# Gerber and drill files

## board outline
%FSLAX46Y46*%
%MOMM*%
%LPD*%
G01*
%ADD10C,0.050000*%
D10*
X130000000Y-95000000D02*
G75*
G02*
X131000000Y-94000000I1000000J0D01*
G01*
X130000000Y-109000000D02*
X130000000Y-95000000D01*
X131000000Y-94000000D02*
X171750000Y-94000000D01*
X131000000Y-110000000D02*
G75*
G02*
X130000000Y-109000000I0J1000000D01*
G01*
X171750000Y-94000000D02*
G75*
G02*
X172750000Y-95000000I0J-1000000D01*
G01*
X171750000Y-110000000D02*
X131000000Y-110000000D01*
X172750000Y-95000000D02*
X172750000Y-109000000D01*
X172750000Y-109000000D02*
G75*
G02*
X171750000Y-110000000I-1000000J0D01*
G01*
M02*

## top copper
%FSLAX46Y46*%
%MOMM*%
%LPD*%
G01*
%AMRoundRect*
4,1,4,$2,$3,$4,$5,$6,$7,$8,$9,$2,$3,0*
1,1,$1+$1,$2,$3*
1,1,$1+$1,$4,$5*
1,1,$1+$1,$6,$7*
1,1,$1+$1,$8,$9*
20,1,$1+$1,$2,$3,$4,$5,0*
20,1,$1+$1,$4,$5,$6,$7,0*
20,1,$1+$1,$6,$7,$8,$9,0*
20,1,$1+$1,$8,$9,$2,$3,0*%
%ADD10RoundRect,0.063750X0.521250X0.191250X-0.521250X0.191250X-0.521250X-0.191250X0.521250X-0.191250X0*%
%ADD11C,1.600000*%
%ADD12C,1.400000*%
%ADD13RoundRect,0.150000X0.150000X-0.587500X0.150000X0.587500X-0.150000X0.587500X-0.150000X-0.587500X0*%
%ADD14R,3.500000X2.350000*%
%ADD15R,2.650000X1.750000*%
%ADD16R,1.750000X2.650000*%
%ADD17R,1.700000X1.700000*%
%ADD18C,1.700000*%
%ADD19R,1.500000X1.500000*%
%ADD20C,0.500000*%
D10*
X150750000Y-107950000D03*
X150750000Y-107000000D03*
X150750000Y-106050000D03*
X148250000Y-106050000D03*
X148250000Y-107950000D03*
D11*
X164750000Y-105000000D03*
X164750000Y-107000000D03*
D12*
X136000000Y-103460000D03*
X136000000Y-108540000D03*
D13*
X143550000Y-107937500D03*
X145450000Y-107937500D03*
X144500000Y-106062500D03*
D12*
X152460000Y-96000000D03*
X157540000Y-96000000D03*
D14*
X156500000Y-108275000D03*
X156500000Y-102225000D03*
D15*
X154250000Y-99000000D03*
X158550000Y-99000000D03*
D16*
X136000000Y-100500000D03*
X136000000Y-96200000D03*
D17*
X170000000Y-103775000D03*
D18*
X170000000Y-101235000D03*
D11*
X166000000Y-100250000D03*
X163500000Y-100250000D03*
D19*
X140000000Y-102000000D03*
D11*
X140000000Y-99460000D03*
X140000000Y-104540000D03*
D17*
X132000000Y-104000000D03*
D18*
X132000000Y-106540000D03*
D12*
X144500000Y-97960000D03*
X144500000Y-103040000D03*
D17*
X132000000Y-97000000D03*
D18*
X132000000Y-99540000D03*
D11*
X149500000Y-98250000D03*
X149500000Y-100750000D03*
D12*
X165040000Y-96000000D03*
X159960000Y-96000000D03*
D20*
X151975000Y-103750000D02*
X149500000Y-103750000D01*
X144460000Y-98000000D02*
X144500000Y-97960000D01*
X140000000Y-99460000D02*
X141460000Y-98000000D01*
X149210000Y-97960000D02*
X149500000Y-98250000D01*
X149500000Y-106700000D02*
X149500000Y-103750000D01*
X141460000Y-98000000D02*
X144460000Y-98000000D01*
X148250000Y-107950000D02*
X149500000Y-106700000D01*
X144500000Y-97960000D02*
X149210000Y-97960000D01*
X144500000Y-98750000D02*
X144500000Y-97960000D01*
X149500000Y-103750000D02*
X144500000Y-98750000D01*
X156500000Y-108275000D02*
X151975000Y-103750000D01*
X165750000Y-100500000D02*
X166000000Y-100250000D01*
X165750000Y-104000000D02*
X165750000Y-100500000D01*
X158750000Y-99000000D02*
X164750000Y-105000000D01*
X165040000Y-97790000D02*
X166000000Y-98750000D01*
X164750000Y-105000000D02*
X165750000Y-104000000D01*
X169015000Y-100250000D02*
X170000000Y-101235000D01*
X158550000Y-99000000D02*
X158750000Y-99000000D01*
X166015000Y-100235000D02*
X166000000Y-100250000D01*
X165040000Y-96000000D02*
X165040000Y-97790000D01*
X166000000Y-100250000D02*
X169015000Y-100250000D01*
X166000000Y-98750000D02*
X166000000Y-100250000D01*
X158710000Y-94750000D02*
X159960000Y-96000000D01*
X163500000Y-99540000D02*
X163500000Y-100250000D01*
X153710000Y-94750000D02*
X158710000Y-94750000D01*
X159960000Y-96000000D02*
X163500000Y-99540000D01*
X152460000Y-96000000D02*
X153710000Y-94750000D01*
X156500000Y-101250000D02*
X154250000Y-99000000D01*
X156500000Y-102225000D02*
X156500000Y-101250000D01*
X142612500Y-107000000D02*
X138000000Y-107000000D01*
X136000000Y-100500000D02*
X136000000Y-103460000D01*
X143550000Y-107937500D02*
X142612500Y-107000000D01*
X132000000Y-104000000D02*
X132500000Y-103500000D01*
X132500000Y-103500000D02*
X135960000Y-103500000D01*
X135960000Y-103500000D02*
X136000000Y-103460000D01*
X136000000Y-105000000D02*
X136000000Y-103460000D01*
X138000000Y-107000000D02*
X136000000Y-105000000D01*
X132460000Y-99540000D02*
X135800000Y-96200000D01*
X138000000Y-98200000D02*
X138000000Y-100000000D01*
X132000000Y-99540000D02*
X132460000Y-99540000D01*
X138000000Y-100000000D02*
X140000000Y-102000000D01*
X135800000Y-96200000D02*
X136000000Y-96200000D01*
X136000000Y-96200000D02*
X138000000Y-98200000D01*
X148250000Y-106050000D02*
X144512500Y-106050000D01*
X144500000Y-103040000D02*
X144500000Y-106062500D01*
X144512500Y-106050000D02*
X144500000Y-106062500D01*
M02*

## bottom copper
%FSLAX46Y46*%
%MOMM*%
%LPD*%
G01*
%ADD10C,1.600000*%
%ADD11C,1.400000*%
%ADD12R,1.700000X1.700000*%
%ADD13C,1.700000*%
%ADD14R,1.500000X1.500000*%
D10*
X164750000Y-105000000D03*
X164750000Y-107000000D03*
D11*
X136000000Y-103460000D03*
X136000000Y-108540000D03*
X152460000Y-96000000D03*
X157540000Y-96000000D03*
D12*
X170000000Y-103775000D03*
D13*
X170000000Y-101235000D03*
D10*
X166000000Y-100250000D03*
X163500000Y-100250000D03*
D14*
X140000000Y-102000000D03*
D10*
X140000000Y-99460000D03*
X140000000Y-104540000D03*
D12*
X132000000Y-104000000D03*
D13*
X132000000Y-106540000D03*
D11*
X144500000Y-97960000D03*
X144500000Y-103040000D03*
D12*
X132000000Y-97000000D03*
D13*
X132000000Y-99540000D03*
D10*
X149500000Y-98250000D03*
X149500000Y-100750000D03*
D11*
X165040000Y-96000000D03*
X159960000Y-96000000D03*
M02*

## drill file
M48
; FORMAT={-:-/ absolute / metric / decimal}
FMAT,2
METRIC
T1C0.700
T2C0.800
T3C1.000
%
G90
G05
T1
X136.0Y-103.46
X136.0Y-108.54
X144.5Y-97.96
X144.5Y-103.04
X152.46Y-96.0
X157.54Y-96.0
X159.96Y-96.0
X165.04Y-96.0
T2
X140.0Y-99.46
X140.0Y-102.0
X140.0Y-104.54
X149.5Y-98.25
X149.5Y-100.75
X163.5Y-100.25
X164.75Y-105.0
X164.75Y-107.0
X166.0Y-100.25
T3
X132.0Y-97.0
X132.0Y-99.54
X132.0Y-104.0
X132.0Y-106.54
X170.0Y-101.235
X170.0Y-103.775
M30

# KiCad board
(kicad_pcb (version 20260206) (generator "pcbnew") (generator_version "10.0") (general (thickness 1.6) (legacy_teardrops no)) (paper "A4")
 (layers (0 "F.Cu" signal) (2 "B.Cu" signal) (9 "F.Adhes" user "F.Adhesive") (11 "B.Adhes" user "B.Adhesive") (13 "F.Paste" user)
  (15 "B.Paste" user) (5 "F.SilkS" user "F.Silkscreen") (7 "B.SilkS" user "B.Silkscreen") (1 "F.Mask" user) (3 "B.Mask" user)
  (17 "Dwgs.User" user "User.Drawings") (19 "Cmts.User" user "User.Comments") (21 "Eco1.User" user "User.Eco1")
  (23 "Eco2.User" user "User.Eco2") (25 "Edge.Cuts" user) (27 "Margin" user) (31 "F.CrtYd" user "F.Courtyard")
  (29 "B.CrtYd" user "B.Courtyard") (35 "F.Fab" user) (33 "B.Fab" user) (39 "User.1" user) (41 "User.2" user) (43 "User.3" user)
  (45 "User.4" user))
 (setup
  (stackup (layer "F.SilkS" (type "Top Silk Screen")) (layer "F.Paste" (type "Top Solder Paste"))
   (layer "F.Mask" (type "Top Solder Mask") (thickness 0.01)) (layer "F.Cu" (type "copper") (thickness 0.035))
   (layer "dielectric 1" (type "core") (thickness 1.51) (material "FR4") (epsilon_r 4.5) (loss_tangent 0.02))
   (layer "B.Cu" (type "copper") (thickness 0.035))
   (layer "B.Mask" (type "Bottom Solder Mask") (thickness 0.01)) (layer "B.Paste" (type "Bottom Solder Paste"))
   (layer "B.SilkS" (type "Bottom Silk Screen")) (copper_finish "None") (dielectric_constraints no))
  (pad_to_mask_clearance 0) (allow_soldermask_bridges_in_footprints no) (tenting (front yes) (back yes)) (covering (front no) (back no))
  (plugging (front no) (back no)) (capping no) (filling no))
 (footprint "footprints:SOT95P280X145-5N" (layer "F.Cu") (at 149.5 107 180)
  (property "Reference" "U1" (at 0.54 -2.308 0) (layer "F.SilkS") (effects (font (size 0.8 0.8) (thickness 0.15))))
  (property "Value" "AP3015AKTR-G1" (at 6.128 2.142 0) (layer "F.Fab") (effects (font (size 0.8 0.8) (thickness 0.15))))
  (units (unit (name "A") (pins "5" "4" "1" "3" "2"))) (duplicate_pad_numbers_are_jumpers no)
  (pad "1" smd roundrect (at -1.25 -0.95 180) (size 1.17 0.51) (layers "F.Cu" "F.Mask" "F.Paste") (roundrect_rratio 0.125)
   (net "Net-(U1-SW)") (solder_mask_margin 0.102))
  (pad "2" smd roundrect (at -1.25 0 180) (size 1.17 0.51) (layers "F.Cu" "F.Mask" "F.Paste") (roundrect_rratio 0.125) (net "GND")
   (solder_mask_margin 0.102))
  (pad "3" smd roundrect (at -1.25 0.95 180) (size 1.17 0.51) (layers "F.Cu" "F.Mask" "F.Paste") (roundrect_rratio 0.125)
   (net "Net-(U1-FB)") (solder_mask_margin 0.102))
  (pad "4" smd roundrect (at 1.25 0.95 180) (size 1.17 0.51) (layers "F.Cu" "F.Mask" "F.Paste") (roundrect_rratio 0.125) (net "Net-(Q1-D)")
   (solder_mask_margin 0.102))
  (pad "5" smd roundrect (at 1.25 -0.95 180) (size 1.17 0.51) (layers "F.Cu" "F.Mask" "F.Paste") (roundrect_rratio 0.125)
   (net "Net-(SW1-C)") (solder_mask_margin 0.102)))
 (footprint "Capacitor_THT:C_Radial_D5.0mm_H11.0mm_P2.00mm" (layer "F.Cu") (at 164.75 105 -90)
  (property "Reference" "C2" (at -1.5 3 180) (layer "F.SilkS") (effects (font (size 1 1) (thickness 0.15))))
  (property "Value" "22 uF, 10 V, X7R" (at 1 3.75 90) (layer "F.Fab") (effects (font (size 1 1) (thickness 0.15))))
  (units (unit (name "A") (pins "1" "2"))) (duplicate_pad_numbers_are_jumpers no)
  (pad "1" thru_hole circle (at 0 0 270) (size 1.6 1.6) (drill 0.8) (layers "*.Cu" "*.Mask") (remove_unused_layers no) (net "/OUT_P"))
  (pad "2" thru_hole circle (at 2 0 270) (size 1.6 1.6) (drill 0.8) (layers "*.Cu" "*.Mask") (remove_unused_layers no) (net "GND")))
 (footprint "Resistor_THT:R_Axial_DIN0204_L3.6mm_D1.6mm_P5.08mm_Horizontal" (layer "F.Cu") (at 136 103.46 -90)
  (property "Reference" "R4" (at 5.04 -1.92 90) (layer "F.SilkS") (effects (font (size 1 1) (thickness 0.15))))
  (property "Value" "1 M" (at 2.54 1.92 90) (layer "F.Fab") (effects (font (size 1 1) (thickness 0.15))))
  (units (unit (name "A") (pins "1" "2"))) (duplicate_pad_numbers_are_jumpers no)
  (pad "1" thru_hole circle (at 0 0 270) (size 1.4 1.4) (drill 0.7) (layers "*.Cu" "*.Mask") (remove_unused_layers no) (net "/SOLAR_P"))
  (pad "2" thru_hole circle (at 5.08 0 270) (size 1.4 1.4) (drill 0.7) (layers "*.Cu" "*.Mask") (remove_unused_layers no) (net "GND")))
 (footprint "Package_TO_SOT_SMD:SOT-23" (layer "F.Cu") (at 144.5 107 90)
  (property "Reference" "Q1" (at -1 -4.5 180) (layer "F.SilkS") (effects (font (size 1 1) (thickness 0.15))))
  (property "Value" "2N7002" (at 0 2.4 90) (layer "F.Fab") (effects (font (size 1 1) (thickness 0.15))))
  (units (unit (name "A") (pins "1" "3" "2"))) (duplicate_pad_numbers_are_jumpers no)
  (pad "1" smd roundrect (at -0.9375 -0.95 90) (size 1.475 0.6) (layers "F.Cu" "F.Mask" "F.Paste") (roundrect_rratio 0.25) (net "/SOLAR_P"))
  (pad "2" smd roundrect (at -0.9375 0.95 90) (size 1.475 0.6) (layers "F.Cu" "F.Mask" "F.Paste") (roundrect_rratio 0.25) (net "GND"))
  (pad "3" smd roundrect (at 0.9375 0 90) (size 1.475 0.6) (layers "F.Cu" "F.Mask" "F.Paste") (roundrect_rratio 0.25) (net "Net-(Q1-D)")))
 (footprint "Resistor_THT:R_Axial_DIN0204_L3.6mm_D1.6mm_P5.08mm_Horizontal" (layer "F.Cu") (at 152.46 96)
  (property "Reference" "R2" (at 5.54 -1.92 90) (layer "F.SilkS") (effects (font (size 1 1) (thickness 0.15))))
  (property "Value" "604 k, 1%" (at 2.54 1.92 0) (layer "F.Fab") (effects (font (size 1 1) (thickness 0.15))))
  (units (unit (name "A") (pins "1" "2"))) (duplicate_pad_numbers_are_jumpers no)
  (pad "1" thru_hole circle (at 0 0) (size 1.4 1.4) (drill 0.7) (layers "*.Cu" "*.Mask") (remove_unused_layers no) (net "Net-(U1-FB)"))
  (pad "2" thru_hole circle (at 5.08 0) (size 1.4 1.4) (drill 0.7) (layers "*.Cu" "*.Mask") (remove_unused_layers no) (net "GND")))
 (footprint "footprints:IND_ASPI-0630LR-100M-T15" (layer "F.Cu") (at 156.5 105.25 90)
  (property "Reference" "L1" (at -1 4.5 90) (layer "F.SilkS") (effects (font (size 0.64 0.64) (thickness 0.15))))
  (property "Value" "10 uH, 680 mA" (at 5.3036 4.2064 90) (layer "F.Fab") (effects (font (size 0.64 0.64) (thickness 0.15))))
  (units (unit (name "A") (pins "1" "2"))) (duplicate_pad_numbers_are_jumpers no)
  (pad "1" smd rect (at -3.025 0 90) (size 2.35 3.5) (layers "F.Cu" "F.Mask" "F.Paste") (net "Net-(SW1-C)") (solder_mask_margin 0.102))
  (pad "2" smd rect (at 3.025 0 90) (size 2.35 3.5) (layers "F.Cu" "F.Mask" "F.Paste") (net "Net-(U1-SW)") (solder_mask_margin 0.102)))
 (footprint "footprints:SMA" (layer "F.Cu") (at 156.25 99)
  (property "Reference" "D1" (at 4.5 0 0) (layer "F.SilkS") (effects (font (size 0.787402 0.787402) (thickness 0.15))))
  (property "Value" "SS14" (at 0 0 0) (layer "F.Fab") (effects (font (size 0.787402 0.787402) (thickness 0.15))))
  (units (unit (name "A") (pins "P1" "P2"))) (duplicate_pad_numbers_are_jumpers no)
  (pad "P1" smd rect (at -2 0) (size 2.65 1.75) (layers "F.Cu" "F.Mask" "F.Paste") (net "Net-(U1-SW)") (solder_mask_margin 0.102))
  (pad "P2" smd rect (at 2.3 0) (size 2.65 1.75) (layers "F.Cu" "F.Mask" "F.Paste") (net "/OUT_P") (solder_mask_margin 0.102)))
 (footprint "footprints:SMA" (layer "F.Cu") (at 136 98.5 90)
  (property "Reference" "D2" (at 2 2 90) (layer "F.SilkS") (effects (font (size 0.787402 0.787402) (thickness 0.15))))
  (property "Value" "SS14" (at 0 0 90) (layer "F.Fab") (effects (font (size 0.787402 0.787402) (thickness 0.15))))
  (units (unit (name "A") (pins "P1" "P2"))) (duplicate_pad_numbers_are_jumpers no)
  (pad "P1" smd rect (at -2 0 90) (size 2.65 1.75) (layers "F.Cu" "F.Mask" "F.Paste") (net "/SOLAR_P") (solder_mask_margin 0.102))
  (pad "P2" smd rect (at 2.3 0 90) (size 2.65 1.75) (layers "F.Cu" "F.Mask" "F.Paste") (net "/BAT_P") (solder_mask_margin 0.102)))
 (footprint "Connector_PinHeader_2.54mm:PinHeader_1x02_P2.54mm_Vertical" (layer "F.Cu") (at 170 103.775 180)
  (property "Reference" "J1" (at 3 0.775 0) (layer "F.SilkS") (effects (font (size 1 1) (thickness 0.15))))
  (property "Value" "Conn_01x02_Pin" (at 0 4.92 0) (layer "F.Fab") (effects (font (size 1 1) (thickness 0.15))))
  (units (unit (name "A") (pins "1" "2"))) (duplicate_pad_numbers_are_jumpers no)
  (pad "1" thru_hole rect (at 0 0 180) (size 1.7 1.7) (drill 1) (layers "*.Cu" "*.Mask") (remove_unused_layers no) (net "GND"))
  (pad "2" thru_hole circle (at 0 2.54 180) (size 1.7 1.7) (drill 1) (layers "*.Cu" "*.Mask") (remove_unused_layers no) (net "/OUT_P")))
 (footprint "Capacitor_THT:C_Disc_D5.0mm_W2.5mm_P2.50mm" (layer "F.Cu") (at 166 100.25 180)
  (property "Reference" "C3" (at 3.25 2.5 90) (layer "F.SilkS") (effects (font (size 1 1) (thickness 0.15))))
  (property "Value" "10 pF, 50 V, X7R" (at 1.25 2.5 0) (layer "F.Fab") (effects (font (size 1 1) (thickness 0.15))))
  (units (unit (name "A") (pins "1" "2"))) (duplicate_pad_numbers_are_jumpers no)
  (pad "1" thru_hole circle (at 0 0 180) (size 1.6 1.6) (drill 0.8) (layers "*.Cu" "*.Mask") (remove_unused_layers no) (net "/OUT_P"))
  (pad "2" thru_hole circle (at 2.5 0 180) (size 1.6 1.6) (drill 0.8) (layers "*.Cu" "*.Mask") (remove_unused_layers no) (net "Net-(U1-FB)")))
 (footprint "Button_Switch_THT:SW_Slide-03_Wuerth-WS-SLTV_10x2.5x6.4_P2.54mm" (layer "F.Cu") (at 140 102 -90)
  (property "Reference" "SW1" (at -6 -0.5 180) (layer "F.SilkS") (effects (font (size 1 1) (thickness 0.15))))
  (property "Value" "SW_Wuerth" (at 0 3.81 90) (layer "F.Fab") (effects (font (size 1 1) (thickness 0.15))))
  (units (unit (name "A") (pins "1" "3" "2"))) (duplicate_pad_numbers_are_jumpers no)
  (pad "1" thru_hole rect (at 0 0 270) (size 1.5 1.5) (drill 0.8) (layers "*.Cu" "*.Mask") (remove_unused_layers no) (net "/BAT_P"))
  (pad "2" thru_hole circle (at -2.54 0 270) (size 1.6 1.6) (drill 0.8) (layers "*.Cu" "*.Mask") (remove_unused_layers no)
   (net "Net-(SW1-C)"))
  (pad "3" thru_hole circle (at 2.54 0 270) (size 1.6 1.6) (drill 0.8) (layers "*.Cu" "*.Mask") (remove_unused_layers no) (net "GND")))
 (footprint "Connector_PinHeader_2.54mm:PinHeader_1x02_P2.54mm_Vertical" (layer "F.Cu") (at 132 104)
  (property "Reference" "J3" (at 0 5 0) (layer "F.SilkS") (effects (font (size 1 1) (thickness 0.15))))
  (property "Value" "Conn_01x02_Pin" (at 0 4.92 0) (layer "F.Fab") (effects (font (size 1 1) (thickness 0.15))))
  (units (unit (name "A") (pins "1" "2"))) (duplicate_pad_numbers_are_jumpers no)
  (pad "1" thru_hole rect (at 0 0) (size 1.7 1.7) (drill 1) (layers "*.Cu" "*.Mask") (remove_unused_layers no) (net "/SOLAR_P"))
  (pad "2" thru_hole circle (at 0 2.54) (size 1.7 1.7) (drill 1) (layers "*.Cu" "*.Mask") (remove_unused_layers no) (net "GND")))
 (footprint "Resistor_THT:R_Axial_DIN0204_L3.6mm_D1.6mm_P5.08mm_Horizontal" (layer "F.Cu") (at 144.5 97.96 -90)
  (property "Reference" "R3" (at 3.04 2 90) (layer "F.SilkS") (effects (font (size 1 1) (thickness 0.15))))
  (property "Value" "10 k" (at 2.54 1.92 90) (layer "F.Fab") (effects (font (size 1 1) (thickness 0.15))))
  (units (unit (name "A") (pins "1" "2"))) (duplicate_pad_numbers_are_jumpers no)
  (pad "1" thru_hole circle (at 0 0 270) (size 1.4 1.4) (drill 0.7) (layers "*.Cu" "*.Mask") (remove_unused_layers no) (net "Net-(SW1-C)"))
  (pad "2" thru_hole circle (at 5.08 0 270) (size 1.4 1.4) (drill 0.7) (layers "*.Cu" "*.Mask") (remove_unused_layers no) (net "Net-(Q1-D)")))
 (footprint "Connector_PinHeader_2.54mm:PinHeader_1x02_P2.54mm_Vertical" (layer "F.Cu") (at 132 97)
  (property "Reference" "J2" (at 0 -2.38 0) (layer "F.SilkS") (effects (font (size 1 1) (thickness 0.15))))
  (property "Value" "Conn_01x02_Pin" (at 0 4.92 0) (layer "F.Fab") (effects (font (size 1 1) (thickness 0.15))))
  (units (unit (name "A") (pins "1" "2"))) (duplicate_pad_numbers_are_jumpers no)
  (pad "1" thru_hole rect (at 0 0) (size 1.7 1.7) (drill 1) (layers "*.Cu" "*.Mask") (remove_unused_layers no) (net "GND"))
  (pad "2" thru_hole circle (at 0 2.54) (size 1.7 1.7) (drill 1) (layers "*.Cu" "*.Mask") (remove_unused_layers no) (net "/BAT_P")))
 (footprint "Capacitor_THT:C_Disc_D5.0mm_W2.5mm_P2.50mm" (layer "F.Cu") (at 149.5 98.25 -90)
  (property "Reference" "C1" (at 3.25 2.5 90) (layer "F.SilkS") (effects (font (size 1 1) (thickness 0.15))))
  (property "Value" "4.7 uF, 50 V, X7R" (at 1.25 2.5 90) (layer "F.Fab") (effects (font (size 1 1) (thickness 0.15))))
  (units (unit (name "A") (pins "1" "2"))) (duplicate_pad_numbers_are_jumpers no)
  (pad "1" thru_hole circle (at 0 0 270) (size 1.6 1.6) (drill 0.8) (layers "*.Cu" "*.Mask") (remove_unused_layers no) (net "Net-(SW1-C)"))
  (pad "2" thru_hole circle (at 2.5 0 270) (size 1.6 1.6) (drill 0.8) (layers "*.Cu" "*.Mask") (remove_unused_layers no) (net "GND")))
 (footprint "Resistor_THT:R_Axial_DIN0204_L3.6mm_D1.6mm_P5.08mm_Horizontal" (layer "F.Cu") (at 165.04 96 180)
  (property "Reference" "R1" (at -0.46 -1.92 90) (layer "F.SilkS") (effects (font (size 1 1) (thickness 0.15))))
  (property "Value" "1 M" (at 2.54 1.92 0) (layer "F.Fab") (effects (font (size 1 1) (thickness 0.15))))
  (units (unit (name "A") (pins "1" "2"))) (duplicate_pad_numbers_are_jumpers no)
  (pad "1" thru_hole circle (at 0 0 180) (size 1.4 1.4) (drill 0.7) (layers "*.Cu" "*.Mask") (remove_unused_layers no) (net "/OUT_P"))
  (pad "2" thru_hole circle (at 5.08 0 180) (size 1.4 1.4) (drill 0.7) (layers "*.Cu" "*.Mask") (remove_unused_layers no)
   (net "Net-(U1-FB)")))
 (gr_arc (start 130 95) (mid 130.292893 94.292893) (end 131 94) (stroke (width 0.05) (type default)) (layer "Edge.Cuts"))
 (gr_line (start 130 109) (end 130 95) (stroke (width 0.05) (type default)) (layer "Edge.Cuts"))
 (gr_line (start 131 94) (end 171.75 94) (stroke (width 0.05) (type default)) (layer "Edge.Cuts"))
 (gr_arc (start 131 110) (mid 130.292893 109.707107) (end 130 109) (stroke (width 0.05) (type default)) (layer "Edge.Cuts"))
 (gr_arc (start 171.75 94) (mid 172.457107 94.292893) (end 172.75 95) (stroke (width 0.05) (type default)) (layer "Edge.Cuts"))
 (gr_line (start 171.75 110) (end 131 110) (stroke (width 0.05) (type default)) (layer "Edge.Cuts"))
 (gr_line (start 172.75 95) (end 172.75 109) (stroke (width 0.05) (type default)) (layer "Edge.Cuts"))
 (gr_arc (start 172.75 109) (mid 172.457107 109.707107) (end 171.75 110) (stroke (width 0.05) (type default)) (layer "Edge.Cuts"))
 (segment (start 151.975 103.75) (end 149.5 103.75) (width 0.5) (layer "F.Cu") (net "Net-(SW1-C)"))
 (segment (start 144.46 98) (end 144.5 97.96) (width 0.5) (layer "F.Cu") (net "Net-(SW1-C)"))
 (segment (start 140 99.46) (end 141.46 98) (width 0.5) (layer "F.Cu") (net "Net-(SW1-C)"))
 (segment (start 149.21 97.96) (end 149.5 98.25) (width 0.5) (layer "F.Cu") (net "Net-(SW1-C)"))
 (segment (start 149.5 106.7) (end 149.5 103.75) (width 0.5) (layer "F.Cu") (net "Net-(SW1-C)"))
 (segment (start 141.46 98) (end 144.46 98) (width 0.5) (layer "F.Cu") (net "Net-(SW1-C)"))
 (segment (start 148.25 107.95) (end 149.5 106.7) (width 0.5) (layer "F.Cu") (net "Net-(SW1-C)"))
 (segment (start 144.5 97.96) (end 149.21 97.96) (width 0.5) (layer "F.Cu") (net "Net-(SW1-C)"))
 (segment (start 144.5 98.75) (end 144.5 97.96) (width 0.5) (layer "F.Cu") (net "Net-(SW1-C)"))
 (segment (start 149.5 103.75) (end 144.5 98.75) (width 0.5) (layer "F.Cu") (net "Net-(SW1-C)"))
 (segment (start 156.5 108.275) (end 151.975 103.75) (width 0.5) (layer "F.Cu") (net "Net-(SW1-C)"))
 (segment (start 165.75 100.5) (end 166 100.25) (width 0.5) (layer "F.Cu") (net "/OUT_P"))
 (segment (start 165.75 104) (end 165.75 100.5) (width 0.5) (layer "F.Cu") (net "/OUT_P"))
 (segment (start 158.75 99) (end 164.75 105) (width 0.5) (layer "F.Cu") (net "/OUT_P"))
 (segment (start 165.04 97.79) (end 166 98.75) (width 0.5) (layer "F.Cu") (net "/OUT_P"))
 (segment (start 164.75 105) (end 165.75 104) (width 0.5) (layer "F.Cu") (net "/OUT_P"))
 (segment (start 169.015 100.25) (end 170 101.235) (width 0.5) (layer "F.Cu") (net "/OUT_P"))
 (segment (start 158.55 99) (end 158.75 99) (width 0.5) (layer "F.Cu") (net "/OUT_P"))
 (segment (start 166.015 100.235) (end 166 100.25) (width 0.5) (layer "F.Cu") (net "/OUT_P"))
 (segment (start 165.04 96) (end 165.04 97.79) (width 0.5) (layer "F.Cu") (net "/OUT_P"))
 (segment (start 166 100.25) (end 169.015 100.25) (width 0.5) (layer "F.Cu") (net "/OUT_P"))
 (segment (start 166 98.75) (end 166 100.25) (width 0.5) (layer "F.Cu") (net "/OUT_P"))
 (segment (start 158.71 94.75) (end 159.96 96) (width 0.5) (layer "F.Cu") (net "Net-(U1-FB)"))
 (segment (start 163.5 99.54) (end 163.5 100.25) (width 0.5) (layer "F.Cu") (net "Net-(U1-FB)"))
 (segment (start 153.71 94.75) (end 158.71 94.75) (width 0.5) (layer "F.Cu") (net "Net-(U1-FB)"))
 (segment (start 159.96 96) (end 163.5 99.54) (width 0.5) (layer "F.Cu") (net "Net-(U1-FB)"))
 (segment (start 152.46 96) (end 153.71 94.75) (width 0.5) (layer "F.Cu") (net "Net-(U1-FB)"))
 (segment (start 156.5 101.25) (end 154.25 99) (width 0.5) (layer "F.Cu") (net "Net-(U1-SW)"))
 (segment (start 156.5 102.225) (end 156.5 101.25) (width 0.5) (layer "F.Cu") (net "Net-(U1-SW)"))
 (segment (start 142.6125 107) (end 138 107) (width 0.5) (layer "F.Cu") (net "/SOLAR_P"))
 (segment (start 136 100.5) (end 136 103.46) (width 0.5) (layer "F.Cu") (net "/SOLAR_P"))
 (segment (start 143.55 107.9375) (end 142.6125 107) (width 0.5) (layer "F.Cu") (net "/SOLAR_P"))
 (segment (start 132 104) (end 132.5 103.5) (width 0.5) (layer "F.Cu") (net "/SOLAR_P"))
 (segment (start 132.5 103.5) (end 135.96 103.5) (width 0.5) (layer "F.Cu") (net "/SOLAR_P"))
 (segment (start 135.96 103.5) (end 136 103.46) (width 0.5) (layer "F.Cu") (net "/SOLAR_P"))
 (segment (start 136 105) (end 136 103.46) (width 0.5) (layer "F.Cu") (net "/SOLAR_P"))
 (segment (start 138 107) (end 136 105) (width 0.5) (layer "F.Cu") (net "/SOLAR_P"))
 (segment (start 132.46 99.54) (end 135.8 96.2) (width 0.5) (layer "F.Cu") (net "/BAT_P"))
 (segment (start 138 98.2) (end 138 100) (width 0.5) (layer "F.Cu") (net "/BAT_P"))
 (segment (start 132 99.54) (end 132.46 99.54) (width 0.5) (layer "F.Cu") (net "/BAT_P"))
 (segment (start 138 100) (end 140 102) (width 0.5) (layer "F.Cu") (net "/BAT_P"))
 (segment (start 135.8 96.2) (end 136 96.2) (width 0.5) (layer "F.Cu") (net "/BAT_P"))
 (segment (start 136 96.2) (end 138 98.2) (width 0.5) (layer "F.Cu") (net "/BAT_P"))
 (segment (start 148.25 106.05) (end 144.5125 106.05) (width 0.5) (layer "F.Cu") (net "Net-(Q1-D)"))
 (segment (start 144.5 103.04) (end 144.5 106.0625) (width 0.5) (layer "F.Cu") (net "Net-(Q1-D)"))
 (segment (start 144.5125 106.05) (end 144.5 106.0625) (width 0.5) (layer "F.Cu") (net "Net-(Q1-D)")))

